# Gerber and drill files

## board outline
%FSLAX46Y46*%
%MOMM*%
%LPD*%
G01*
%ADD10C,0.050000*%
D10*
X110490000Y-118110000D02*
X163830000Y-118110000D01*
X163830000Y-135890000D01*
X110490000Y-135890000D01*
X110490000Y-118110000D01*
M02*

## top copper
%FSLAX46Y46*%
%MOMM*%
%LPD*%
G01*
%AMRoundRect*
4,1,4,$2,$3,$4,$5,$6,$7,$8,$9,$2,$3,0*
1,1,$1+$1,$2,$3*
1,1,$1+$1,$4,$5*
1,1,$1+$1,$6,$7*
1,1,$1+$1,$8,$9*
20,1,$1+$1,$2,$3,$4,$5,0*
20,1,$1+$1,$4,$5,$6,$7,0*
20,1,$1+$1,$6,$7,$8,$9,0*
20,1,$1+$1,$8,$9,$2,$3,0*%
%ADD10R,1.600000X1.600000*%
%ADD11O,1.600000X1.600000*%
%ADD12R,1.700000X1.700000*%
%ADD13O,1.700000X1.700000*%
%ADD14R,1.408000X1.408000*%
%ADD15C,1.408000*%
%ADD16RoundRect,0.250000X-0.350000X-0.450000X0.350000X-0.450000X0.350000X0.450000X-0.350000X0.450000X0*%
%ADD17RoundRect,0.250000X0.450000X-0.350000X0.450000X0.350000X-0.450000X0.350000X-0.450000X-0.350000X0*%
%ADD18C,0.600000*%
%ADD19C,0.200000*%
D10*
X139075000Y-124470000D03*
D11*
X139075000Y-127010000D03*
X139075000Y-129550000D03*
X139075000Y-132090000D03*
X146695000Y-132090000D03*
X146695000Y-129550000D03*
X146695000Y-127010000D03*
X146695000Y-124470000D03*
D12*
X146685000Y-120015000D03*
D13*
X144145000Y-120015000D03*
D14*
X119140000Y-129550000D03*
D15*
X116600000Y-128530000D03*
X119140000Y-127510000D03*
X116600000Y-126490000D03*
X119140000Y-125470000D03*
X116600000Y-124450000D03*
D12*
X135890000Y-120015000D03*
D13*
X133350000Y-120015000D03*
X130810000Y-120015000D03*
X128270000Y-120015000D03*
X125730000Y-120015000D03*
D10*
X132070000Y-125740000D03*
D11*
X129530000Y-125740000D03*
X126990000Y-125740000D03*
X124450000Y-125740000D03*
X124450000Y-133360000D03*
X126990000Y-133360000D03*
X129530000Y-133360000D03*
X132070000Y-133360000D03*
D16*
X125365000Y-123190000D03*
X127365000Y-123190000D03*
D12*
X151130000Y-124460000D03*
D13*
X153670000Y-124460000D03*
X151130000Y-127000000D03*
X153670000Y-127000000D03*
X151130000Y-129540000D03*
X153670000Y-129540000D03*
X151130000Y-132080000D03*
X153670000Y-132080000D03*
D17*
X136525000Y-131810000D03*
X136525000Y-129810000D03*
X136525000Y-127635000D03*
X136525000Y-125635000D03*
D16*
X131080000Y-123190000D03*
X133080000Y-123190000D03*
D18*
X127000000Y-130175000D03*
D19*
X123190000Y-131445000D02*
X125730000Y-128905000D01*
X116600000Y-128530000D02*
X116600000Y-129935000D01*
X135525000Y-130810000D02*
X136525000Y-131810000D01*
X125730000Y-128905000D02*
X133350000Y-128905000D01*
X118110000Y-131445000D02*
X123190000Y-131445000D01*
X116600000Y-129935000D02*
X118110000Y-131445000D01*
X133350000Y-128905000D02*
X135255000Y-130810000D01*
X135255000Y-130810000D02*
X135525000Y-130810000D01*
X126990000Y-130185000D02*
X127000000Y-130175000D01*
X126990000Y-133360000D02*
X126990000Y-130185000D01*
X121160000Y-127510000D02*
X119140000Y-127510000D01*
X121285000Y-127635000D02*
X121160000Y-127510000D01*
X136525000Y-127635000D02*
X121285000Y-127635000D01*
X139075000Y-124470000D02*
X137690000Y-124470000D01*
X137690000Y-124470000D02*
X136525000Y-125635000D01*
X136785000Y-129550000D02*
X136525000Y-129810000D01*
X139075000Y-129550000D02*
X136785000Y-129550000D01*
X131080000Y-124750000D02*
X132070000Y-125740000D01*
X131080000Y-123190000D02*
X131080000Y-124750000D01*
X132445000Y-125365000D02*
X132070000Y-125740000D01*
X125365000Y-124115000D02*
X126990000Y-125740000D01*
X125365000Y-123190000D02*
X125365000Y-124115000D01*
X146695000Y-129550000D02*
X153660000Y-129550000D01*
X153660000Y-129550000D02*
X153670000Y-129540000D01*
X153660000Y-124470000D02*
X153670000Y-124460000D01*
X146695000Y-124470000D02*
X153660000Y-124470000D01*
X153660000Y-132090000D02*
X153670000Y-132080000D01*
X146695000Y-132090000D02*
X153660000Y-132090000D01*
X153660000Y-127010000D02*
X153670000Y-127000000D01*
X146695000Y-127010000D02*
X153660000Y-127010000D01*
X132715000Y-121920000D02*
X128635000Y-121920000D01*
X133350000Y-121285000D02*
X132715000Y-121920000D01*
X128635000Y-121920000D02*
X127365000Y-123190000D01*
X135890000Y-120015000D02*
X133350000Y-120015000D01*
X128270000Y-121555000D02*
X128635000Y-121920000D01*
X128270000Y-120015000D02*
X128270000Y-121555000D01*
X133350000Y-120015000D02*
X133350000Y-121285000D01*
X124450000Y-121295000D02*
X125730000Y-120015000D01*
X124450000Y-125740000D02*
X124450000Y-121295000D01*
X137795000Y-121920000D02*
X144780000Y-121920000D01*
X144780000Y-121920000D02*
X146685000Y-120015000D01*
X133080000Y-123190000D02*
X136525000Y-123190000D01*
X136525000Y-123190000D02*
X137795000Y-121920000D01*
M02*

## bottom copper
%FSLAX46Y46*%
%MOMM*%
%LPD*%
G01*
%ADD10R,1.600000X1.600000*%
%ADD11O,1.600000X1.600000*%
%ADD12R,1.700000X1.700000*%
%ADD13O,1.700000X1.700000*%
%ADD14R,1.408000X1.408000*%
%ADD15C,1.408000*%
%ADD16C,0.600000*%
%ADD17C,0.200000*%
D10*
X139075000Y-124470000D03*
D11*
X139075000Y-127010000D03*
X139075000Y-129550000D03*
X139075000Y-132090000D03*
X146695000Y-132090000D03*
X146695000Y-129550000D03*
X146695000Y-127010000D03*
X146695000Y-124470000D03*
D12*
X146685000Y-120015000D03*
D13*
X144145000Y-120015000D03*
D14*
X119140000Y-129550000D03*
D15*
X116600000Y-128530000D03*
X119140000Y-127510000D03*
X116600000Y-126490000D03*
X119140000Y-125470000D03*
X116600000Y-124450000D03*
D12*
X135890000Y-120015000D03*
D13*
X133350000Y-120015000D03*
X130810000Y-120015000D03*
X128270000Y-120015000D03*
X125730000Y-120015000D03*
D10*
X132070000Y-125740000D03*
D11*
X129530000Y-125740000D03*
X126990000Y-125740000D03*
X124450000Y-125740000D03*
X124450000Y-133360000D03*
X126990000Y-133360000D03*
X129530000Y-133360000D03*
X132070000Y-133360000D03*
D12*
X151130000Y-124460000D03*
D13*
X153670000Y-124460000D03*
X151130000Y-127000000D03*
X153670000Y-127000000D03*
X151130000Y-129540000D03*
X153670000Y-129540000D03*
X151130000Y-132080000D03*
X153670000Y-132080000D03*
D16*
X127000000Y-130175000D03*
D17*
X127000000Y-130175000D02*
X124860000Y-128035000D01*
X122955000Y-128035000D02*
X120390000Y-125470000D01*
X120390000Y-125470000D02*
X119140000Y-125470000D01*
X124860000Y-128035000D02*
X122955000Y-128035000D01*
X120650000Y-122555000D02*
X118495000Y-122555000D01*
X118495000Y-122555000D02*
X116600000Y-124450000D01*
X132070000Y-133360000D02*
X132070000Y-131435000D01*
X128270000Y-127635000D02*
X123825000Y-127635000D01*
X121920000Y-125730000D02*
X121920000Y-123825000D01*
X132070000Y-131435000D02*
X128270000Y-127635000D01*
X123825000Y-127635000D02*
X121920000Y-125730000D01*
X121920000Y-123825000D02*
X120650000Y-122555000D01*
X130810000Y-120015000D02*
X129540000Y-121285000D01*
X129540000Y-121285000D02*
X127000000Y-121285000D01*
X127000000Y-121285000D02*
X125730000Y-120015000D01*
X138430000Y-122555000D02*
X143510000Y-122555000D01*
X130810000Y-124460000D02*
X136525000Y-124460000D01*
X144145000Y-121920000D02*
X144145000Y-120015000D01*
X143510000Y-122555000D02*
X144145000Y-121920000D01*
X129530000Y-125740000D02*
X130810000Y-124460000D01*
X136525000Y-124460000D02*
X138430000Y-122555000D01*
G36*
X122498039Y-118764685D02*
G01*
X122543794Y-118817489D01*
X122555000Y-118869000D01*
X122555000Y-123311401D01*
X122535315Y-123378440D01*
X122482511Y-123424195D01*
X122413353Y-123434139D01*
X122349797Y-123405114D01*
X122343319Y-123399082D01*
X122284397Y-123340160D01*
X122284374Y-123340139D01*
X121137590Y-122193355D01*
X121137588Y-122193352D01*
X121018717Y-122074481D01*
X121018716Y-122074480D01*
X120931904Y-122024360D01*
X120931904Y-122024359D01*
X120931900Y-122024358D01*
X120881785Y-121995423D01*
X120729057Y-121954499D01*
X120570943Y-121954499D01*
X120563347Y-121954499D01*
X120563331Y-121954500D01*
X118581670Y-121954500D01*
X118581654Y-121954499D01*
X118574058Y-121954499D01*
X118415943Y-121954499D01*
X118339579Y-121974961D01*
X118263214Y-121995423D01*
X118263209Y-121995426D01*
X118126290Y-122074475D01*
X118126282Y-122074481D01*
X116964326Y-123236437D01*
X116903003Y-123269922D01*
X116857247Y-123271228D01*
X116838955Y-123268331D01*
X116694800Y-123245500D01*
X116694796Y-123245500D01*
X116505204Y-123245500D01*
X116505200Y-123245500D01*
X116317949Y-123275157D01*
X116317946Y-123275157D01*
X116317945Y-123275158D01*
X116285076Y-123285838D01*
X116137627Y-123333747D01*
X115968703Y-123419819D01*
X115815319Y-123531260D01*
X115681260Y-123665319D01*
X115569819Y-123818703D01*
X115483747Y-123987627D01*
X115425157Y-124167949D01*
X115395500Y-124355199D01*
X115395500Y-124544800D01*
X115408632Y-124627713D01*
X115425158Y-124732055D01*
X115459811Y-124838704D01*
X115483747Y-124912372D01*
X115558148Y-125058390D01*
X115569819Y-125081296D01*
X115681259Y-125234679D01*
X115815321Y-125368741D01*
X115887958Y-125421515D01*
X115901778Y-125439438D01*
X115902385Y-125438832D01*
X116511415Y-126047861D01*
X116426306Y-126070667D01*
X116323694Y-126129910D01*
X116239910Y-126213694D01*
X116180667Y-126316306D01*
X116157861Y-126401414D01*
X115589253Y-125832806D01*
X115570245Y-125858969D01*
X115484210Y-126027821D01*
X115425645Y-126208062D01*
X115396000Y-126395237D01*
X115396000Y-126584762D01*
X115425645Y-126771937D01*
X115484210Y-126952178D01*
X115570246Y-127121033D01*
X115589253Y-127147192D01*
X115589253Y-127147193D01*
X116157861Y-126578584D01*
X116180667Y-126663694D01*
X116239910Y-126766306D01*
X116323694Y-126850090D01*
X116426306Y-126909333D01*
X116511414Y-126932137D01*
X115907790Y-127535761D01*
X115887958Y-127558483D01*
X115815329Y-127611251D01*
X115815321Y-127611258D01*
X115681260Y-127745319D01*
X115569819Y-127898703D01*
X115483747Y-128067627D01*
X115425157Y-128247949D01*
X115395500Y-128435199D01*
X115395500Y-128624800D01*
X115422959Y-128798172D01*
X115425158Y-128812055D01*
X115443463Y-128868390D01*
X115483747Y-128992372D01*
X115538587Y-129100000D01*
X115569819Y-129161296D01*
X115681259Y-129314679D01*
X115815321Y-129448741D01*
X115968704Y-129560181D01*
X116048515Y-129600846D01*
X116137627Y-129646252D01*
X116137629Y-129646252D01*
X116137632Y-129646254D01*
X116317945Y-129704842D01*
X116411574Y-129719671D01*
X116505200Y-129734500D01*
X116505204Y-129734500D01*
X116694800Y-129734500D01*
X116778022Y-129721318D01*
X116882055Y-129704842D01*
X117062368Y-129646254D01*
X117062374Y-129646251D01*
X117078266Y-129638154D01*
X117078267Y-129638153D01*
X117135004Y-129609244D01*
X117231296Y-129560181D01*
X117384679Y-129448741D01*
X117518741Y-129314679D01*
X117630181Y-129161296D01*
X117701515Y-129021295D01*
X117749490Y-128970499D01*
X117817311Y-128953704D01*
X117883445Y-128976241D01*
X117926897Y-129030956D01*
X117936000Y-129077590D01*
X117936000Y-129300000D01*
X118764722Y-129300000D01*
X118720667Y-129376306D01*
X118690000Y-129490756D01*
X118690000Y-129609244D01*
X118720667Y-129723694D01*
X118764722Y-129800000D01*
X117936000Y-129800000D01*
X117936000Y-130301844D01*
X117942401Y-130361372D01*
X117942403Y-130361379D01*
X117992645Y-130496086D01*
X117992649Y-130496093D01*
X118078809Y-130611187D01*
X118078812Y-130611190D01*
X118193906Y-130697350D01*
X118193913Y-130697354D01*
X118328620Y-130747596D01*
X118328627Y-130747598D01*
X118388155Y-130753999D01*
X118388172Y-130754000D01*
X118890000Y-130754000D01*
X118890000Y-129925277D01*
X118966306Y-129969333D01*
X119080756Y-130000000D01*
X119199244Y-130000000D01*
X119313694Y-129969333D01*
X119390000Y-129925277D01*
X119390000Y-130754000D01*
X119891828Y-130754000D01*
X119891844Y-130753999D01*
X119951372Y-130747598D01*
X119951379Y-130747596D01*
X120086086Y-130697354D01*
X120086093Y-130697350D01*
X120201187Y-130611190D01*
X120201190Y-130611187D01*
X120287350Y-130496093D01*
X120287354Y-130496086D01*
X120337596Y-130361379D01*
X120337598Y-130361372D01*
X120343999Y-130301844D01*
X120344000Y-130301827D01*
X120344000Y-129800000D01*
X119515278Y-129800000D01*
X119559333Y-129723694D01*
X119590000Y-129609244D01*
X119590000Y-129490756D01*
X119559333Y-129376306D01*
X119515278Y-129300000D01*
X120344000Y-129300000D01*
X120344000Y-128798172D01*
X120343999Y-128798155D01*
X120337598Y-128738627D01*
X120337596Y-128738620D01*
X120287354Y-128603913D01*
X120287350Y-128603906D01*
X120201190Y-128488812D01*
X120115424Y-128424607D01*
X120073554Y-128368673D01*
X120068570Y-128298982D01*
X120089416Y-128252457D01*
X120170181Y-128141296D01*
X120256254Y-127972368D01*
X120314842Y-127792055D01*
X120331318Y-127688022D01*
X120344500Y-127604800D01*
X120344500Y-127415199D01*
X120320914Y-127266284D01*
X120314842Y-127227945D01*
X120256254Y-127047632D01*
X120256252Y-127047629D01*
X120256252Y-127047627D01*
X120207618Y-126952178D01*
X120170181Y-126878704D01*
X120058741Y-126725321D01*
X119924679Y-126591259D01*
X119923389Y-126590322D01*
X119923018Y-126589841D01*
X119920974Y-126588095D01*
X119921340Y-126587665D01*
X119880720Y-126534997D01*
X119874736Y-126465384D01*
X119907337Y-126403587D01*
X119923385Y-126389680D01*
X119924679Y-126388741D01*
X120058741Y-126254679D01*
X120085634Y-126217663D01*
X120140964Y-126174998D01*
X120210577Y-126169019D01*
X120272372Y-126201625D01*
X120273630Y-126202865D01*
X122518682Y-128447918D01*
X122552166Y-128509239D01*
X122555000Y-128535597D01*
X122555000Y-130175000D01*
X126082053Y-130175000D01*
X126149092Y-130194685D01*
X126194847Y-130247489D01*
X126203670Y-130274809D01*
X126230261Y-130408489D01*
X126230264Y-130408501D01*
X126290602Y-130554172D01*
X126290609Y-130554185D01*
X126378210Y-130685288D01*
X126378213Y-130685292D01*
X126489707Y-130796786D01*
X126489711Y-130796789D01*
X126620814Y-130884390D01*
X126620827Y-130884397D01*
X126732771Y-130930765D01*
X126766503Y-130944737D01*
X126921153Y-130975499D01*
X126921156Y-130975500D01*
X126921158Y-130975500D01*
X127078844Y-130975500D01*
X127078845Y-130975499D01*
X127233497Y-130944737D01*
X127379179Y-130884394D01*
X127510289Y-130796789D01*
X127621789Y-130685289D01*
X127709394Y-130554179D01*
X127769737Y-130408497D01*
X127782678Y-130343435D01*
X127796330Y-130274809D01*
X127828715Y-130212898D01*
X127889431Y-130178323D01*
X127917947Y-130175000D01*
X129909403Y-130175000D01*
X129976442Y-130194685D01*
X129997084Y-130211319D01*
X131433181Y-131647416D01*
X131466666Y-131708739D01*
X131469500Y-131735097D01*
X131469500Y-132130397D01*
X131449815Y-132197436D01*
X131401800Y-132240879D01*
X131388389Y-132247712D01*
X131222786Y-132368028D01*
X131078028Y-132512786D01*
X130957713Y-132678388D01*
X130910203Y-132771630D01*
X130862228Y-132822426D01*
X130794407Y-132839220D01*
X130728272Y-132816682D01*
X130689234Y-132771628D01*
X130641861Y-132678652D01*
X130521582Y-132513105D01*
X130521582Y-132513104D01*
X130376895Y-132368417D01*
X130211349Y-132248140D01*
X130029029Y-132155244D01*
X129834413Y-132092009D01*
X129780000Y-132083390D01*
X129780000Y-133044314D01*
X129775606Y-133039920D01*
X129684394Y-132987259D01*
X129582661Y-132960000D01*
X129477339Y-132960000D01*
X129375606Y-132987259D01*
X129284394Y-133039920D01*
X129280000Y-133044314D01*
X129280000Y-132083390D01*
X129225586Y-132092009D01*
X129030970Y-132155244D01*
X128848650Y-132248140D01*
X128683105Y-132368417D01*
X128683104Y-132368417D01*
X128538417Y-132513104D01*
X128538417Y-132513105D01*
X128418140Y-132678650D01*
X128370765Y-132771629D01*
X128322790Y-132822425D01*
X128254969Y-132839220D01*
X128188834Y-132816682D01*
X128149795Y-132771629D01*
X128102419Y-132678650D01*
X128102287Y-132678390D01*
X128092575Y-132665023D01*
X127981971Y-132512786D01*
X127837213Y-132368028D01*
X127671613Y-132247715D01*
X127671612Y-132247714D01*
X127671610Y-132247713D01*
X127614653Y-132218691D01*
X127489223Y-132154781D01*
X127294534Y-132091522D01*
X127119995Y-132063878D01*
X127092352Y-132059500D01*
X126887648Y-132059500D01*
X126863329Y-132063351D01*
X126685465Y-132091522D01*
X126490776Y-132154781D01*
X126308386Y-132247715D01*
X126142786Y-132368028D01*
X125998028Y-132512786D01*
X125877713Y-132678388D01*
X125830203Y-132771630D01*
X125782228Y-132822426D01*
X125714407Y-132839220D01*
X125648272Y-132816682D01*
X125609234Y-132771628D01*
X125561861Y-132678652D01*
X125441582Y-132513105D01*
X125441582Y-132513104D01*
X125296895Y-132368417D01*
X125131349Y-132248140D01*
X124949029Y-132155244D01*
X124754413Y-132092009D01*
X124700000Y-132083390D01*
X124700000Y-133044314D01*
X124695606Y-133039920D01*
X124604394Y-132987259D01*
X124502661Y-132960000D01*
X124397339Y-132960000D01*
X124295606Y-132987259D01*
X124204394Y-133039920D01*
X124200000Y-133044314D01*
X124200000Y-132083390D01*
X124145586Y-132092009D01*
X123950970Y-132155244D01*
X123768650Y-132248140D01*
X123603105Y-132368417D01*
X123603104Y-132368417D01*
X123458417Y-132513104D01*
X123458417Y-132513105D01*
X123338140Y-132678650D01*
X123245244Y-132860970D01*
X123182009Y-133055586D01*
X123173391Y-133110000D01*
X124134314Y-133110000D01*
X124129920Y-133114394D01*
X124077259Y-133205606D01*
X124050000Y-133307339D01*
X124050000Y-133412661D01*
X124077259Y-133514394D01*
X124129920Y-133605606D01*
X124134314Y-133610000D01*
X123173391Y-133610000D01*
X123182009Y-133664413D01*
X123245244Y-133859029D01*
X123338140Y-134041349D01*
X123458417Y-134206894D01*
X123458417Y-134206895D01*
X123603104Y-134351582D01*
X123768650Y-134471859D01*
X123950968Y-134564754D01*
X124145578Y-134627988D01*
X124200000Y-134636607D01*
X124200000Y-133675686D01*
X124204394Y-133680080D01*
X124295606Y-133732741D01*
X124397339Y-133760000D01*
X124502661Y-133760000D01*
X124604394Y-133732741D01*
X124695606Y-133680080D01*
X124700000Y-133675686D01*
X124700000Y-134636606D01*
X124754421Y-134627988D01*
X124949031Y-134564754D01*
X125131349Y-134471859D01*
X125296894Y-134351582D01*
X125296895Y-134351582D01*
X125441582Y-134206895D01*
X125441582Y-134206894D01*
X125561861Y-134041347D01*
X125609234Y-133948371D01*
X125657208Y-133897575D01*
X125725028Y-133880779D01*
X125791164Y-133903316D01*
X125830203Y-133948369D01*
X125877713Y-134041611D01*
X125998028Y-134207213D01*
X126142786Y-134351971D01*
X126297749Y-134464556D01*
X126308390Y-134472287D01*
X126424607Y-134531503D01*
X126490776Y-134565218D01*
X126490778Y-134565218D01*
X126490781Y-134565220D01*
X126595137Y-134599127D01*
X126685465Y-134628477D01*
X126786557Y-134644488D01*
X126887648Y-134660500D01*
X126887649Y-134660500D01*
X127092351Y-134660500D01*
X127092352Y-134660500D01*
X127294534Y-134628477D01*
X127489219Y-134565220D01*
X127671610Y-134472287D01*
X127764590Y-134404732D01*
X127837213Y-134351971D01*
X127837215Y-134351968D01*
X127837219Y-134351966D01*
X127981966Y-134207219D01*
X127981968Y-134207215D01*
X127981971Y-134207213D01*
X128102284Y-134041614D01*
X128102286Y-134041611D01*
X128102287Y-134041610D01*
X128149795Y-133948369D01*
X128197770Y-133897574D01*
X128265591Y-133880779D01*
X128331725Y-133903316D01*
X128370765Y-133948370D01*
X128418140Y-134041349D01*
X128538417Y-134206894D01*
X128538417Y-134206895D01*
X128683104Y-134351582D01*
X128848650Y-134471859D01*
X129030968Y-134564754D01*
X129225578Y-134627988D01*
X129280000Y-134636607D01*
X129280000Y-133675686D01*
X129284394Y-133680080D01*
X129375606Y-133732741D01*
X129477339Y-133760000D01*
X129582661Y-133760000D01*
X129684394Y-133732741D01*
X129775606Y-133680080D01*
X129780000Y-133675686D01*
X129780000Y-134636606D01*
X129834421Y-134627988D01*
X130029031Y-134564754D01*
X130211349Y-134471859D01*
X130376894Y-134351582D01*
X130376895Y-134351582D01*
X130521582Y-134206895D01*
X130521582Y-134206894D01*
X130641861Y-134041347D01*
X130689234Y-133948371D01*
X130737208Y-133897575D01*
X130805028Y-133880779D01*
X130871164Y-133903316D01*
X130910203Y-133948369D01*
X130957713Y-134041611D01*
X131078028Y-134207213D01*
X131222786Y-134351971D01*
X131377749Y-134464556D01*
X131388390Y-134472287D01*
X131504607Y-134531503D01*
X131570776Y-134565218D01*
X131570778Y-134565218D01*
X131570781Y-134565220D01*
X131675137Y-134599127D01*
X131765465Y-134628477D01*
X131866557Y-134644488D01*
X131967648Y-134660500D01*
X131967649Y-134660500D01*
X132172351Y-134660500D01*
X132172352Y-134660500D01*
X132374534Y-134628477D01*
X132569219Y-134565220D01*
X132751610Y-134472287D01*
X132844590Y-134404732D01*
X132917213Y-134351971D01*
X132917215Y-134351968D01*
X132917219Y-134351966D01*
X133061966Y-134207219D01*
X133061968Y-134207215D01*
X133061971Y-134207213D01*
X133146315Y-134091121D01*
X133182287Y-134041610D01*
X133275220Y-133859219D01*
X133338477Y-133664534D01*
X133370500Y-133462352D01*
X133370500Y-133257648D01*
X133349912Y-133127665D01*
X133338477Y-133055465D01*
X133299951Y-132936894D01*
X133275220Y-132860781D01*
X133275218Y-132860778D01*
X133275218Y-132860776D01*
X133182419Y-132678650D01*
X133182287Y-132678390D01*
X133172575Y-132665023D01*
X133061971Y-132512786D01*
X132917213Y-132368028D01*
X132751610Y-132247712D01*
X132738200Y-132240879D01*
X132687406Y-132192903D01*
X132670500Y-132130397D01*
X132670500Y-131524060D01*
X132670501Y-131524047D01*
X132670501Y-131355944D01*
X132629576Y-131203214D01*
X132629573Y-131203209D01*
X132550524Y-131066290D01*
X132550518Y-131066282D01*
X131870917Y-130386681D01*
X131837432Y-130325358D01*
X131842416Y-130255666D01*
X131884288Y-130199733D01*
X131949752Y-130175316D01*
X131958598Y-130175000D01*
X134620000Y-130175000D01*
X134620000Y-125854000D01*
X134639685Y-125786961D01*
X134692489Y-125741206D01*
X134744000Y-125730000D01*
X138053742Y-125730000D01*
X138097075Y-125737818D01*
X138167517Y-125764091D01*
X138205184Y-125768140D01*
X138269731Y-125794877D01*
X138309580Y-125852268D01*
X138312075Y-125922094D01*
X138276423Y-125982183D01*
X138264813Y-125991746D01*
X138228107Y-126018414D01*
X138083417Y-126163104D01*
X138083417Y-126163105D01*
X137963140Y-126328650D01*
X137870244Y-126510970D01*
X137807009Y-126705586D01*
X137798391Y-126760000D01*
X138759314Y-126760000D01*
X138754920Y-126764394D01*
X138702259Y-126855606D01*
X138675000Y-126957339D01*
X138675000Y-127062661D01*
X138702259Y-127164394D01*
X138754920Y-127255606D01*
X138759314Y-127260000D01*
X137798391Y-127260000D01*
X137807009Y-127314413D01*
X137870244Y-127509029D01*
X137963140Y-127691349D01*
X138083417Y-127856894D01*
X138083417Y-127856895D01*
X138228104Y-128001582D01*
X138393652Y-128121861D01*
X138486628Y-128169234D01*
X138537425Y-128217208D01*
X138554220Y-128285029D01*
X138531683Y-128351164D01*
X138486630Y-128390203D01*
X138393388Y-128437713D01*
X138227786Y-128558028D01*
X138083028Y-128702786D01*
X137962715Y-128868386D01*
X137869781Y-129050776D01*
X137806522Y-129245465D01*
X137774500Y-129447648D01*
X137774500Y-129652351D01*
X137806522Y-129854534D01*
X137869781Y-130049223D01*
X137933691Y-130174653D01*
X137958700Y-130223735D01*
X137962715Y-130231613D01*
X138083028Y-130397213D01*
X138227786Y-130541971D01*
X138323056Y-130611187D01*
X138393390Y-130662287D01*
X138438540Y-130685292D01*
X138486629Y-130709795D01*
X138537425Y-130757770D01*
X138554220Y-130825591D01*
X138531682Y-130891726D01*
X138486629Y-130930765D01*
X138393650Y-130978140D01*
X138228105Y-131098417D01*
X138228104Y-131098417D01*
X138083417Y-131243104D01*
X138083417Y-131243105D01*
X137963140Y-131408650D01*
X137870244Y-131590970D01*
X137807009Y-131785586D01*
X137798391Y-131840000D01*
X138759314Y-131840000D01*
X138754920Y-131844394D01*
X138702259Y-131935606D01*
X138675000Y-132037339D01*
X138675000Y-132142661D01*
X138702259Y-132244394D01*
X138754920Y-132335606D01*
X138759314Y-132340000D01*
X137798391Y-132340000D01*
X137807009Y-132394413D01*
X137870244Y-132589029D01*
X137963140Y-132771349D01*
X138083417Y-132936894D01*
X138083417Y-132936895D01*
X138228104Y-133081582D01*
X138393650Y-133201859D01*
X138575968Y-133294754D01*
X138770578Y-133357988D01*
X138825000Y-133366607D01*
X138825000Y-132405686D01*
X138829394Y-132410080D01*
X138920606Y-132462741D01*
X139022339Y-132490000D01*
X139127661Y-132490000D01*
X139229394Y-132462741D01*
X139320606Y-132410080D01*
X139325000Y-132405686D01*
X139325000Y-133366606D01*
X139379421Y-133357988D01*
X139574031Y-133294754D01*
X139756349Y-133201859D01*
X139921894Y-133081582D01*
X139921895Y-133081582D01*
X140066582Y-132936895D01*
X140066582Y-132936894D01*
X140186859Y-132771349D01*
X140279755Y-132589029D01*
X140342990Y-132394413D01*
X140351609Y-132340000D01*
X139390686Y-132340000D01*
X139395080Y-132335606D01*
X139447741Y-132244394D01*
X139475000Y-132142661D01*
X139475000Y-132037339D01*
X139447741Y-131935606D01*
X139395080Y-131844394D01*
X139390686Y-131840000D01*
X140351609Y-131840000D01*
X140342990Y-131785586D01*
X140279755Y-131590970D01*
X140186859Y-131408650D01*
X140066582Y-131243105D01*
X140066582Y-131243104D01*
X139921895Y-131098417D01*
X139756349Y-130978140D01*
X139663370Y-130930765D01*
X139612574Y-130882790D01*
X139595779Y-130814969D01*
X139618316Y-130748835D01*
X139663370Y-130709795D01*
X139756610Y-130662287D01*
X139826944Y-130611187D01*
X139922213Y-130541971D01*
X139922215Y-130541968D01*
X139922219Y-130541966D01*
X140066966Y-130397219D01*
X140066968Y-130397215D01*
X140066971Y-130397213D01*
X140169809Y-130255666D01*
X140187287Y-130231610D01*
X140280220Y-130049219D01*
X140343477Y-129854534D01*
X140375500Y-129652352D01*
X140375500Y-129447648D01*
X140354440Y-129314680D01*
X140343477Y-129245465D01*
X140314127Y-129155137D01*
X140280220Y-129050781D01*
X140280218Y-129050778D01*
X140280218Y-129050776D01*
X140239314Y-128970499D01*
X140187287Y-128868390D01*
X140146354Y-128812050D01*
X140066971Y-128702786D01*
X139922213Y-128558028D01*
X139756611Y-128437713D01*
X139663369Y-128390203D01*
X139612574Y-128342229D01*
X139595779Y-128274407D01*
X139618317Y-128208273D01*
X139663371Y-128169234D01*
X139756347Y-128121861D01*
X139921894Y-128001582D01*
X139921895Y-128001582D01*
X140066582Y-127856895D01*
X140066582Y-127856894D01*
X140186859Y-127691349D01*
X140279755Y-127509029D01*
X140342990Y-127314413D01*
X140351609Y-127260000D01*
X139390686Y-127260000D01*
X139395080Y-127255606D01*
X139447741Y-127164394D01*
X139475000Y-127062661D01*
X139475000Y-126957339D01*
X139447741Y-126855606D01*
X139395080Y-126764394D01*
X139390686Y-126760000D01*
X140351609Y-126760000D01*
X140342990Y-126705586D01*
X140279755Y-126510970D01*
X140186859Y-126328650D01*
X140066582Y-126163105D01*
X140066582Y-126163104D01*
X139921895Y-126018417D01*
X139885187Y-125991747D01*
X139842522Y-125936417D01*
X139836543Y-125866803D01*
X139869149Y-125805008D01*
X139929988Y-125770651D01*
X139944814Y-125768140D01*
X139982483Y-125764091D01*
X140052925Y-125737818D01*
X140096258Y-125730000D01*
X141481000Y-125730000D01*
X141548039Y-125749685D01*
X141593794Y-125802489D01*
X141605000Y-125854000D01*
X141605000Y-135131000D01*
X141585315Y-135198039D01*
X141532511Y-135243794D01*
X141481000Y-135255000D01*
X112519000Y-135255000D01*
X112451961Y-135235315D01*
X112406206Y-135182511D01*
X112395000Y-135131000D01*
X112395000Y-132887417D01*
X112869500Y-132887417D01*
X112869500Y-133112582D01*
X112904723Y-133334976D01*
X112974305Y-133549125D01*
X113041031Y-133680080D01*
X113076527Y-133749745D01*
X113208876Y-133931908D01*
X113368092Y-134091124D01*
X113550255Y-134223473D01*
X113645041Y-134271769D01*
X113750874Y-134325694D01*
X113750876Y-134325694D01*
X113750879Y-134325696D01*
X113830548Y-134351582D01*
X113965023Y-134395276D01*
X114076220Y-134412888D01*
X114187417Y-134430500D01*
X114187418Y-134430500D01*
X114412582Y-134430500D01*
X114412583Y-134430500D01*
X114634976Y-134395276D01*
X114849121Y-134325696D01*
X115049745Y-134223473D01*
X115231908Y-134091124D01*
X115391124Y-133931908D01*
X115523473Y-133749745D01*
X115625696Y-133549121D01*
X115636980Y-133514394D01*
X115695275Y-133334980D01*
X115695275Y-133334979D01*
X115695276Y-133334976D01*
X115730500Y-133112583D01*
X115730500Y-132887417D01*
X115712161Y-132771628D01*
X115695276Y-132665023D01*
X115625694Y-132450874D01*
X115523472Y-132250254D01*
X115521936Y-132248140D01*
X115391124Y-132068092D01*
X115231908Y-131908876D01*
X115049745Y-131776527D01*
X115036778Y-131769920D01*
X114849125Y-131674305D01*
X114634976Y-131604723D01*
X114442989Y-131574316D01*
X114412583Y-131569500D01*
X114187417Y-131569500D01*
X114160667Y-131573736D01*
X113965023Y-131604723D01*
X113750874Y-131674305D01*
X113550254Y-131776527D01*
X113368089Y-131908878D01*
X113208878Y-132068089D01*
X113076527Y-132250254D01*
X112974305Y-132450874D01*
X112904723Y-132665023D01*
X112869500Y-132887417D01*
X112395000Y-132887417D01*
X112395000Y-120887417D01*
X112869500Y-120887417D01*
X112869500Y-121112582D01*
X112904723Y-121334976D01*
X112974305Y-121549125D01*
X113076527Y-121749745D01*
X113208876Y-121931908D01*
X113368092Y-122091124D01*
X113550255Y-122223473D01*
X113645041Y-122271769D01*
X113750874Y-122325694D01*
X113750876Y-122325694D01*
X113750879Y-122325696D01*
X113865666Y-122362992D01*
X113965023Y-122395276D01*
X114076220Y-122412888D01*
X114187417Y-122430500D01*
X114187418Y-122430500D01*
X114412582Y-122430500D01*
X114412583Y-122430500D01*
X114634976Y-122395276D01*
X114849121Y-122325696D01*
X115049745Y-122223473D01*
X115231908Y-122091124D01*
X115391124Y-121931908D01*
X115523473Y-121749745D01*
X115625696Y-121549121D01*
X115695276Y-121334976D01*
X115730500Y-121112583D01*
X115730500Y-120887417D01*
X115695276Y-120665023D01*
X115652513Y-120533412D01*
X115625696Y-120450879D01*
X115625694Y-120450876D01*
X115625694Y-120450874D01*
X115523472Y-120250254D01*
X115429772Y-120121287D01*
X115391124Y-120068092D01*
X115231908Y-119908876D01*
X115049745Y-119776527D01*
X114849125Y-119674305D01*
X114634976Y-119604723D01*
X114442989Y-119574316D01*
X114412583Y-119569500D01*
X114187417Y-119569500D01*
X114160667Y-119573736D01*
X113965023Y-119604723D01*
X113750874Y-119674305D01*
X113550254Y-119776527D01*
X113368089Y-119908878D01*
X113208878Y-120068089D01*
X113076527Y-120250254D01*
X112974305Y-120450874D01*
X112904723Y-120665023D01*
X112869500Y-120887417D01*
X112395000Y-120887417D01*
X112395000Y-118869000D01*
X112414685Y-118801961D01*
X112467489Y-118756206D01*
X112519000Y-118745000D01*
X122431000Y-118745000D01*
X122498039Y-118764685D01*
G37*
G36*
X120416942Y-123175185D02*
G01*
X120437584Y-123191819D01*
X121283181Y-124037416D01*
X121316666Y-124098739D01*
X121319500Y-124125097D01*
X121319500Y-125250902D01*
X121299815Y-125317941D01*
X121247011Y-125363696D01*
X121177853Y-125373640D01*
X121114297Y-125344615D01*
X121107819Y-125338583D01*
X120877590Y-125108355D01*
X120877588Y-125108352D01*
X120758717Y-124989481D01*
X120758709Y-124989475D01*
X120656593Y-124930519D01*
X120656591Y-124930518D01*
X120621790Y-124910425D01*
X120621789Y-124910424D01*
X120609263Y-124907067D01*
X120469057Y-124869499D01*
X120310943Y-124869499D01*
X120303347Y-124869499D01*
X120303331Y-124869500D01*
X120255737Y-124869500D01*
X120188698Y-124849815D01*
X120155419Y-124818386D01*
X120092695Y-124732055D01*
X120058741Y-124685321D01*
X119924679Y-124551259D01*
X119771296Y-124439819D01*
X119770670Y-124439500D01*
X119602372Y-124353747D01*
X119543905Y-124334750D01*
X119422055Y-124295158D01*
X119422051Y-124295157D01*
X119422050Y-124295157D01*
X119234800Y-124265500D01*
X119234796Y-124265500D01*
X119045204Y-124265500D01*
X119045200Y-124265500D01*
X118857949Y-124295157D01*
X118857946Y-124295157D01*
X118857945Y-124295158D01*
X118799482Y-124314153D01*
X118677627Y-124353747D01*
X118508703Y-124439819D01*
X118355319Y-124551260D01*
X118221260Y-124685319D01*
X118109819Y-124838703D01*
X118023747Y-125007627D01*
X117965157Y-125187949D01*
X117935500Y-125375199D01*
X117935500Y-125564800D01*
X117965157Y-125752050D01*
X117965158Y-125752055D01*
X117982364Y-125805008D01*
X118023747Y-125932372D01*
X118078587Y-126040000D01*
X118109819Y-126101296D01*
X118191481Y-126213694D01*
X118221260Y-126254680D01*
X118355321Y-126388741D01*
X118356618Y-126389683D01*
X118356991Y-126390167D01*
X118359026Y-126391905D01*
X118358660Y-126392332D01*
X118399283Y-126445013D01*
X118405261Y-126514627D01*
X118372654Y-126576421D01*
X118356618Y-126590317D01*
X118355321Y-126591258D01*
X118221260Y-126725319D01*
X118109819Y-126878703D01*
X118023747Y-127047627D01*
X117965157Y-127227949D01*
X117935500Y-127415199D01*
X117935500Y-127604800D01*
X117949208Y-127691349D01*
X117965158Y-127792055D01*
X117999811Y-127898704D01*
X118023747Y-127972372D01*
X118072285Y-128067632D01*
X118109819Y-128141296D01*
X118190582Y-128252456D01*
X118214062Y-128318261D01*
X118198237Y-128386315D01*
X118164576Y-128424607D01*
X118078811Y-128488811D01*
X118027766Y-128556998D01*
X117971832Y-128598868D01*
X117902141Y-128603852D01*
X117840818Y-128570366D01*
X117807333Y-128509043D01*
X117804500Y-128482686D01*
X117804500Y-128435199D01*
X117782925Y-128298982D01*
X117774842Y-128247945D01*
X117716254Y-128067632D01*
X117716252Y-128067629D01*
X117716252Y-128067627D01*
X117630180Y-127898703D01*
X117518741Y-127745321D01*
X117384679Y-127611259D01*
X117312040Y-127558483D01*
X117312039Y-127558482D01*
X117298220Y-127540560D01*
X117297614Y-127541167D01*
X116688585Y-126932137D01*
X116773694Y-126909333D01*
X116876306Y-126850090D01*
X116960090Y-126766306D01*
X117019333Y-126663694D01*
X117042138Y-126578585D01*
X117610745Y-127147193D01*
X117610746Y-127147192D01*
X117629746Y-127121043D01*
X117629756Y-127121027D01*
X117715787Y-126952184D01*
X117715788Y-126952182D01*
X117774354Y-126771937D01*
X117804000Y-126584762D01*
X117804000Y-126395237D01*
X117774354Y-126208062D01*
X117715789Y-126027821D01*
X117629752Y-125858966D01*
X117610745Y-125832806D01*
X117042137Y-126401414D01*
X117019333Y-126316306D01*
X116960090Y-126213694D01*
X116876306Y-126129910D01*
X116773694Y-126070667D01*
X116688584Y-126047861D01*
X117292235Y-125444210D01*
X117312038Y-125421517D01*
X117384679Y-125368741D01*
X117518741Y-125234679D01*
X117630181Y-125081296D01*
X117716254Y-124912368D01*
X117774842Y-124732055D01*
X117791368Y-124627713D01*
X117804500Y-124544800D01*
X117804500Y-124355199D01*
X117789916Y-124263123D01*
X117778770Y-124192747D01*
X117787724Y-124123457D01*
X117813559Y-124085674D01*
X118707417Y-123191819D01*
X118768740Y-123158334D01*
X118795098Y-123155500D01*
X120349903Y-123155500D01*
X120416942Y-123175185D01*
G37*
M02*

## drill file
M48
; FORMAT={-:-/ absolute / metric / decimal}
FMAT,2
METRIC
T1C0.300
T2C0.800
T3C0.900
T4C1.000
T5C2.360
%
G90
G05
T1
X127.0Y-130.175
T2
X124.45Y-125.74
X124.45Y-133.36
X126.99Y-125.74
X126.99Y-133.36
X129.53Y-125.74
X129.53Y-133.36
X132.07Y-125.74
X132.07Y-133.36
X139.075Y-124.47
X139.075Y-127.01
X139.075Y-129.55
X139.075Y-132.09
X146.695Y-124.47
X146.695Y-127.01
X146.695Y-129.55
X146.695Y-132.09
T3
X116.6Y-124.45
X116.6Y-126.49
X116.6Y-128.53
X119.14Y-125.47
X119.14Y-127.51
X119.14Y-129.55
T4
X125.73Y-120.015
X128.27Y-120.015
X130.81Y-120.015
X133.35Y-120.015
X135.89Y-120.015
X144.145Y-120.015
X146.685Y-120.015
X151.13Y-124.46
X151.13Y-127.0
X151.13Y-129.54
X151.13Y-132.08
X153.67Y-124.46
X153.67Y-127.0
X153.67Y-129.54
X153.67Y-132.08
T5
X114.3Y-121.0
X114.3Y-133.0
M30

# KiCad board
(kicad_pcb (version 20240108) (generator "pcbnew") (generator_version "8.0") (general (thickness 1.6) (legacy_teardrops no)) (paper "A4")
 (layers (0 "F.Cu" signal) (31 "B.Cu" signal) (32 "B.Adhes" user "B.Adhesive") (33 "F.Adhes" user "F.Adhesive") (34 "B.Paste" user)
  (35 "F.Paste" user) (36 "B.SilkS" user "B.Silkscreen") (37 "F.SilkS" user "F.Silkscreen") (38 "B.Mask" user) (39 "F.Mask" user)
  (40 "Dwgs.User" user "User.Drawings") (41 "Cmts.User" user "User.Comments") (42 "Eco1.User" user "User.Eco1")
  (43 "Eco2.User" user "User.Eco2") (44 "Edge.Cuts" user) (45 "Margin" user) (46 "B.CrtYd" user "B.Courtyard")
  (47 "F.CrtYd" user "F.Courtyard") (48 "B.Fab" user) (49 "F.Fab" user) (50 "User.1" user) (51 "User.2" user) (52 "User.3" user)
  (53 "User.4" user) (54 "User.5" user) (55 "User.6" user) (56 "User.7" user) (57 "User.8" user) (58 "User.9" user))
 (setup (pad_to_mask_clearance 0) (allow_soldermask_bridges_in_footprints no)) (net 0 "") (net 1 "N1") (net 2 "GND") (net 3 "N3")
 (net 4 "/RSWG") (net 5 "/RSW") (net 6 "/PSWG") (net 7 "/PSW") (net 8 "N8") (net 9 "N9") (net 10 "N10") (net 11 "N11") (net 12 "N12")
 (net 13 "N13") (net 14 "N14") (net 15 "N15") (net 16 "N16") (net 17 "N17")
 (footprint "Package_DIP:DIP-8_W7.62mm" (layer "F.Cu") (at 139.075 124.47)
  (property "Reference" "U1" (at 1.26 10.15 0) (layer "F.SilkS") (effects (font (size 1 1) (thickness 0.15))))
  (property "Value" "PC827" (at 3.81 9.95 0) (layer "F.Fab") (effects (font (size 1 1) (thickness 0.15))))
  (pad "1" thru_hole rect (at 0 0) (size 1.6 1.6) (drill 0.8) (layers "*.Cu" "*.Mask") (remove_unused_layers no) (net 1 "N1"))
  (pad "2" thru_hole oval (at 0 2.54) (size 1.6 1.6) (drill 0.8) (layers "*.Cu" "*.Mask") (remove_unused_layers no) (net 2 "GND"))
  (pad "3" thru_hole oval (at 0 5.08) (size 1.6 1.6) (drill 0.8) (layers "*.Cu" "*.Mask") (remove_unused_layers no) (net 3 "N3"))
  (pad "4" thru_hole oval (at 0 7.62) (size 1.6 1.6) (drill 0.8) (layers "*.Cu" "*.Mask") (remove_unused_layers no) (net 2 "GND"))
  (pad "5" thru_hole oval (at 7.62 7.62) (size 1.6 1.6) (drill 0.8) (layers "*.Cu" "*.Mask") (remove_unused_layers no) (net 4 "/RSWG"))
  (pad "6" thru_hole oval (at 7.62 5.08) (size 1.6 1.6) (drill 0.8) (layers "*.Cu" "*.Mask") (remove_unused_layers no) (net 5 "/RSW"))
  (pad "7" thru_hole oval (at 7.62 2.54) (size 1.6 1.6) (drill 0.8) (layers "*.Cu" "*.Mask") (remove_unused_layers no) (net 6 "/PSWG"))
  (pad "8" thru_hole oval (at 7.62 0) (size 1.6 1.6) (drill 0.8) (layers "*.Cu" "*.Mask") (remove_unused_layers no) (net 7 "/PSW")))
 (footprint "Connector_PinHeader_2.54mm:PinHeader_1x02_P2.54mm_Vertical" (layer "F.Cu") (at 146.685 120.015 -90)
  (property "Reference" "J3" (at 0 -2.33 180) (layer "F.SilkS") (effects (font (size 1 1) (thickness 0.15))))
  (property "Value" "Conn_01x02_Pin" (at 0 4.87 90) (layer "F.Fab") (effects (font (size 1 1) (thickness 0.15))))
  (pad "1" thru_hole rect (at 0 0 270) (size 1.7 1.7) (drill 1) (layers "*.Cu" "*.Mask") (remove_unused_layers no) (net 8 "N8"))
  (pad "2" thru_hole oval (at 0 2.54 270) (size 1.7 1.7) (drill 1) (layers "*.Cu" "*.Mask") (remove_unused_layers no) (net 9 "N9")))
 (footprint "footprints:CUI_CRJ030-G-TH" (layer "F.Cu") (at 114.3 127 -90)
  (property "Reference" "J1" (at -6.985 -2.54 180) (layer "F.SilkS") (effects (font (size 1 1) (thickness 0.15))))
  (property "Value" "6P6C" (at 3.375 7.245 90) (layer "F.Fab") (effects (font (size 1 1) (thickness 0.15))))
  (pad "" np_thru_hole circle (at -6 0 270) (size 2.36 2.36) (drill 2.36) (layers "*.Cu" "*.Mask"))
  (pad "" np_thru_hole circle (at 6 0 270) (size 2.36 2.36) (drill 2.36) (layers "*.Cu" "*.Mask"))
  (pad "1" thru_hole rect (at 2.55 -4.84 270) (size 1.408 1.408) (drill 0.9) (layers "*.Cu" "*.Mask") (remove_unused_layers no)
   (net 2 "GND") (solder_mask_margin 0.102))
  (pad "2" thru_hole circle (at 1.53 -2.3 270) (size 1.408 1.408) (drill 0.9) (layers "*.Cu" "*.Mask") (remove_unused_layers no)
   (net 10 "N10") (solder_mask_margin 0.102))
  (pad "3" thru_hole circle (at 0.51 -4.84 270) (size 1.408 1.408) (drill 0.9) (layers "*.Cu" "*.Mask") (remove_unused_layers no)
   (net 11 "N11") (solder_mask_margin 0.102))
  (pad "4" thru_hole circle (at -0.51 -2.3 270) (size 1.408 1.408) (drill 0.9) (layers "*.Cu" "*.Mask") (remove_unused_layers no)
   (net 2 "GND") (solder_mask_margin 0.102))
  (pad "5" thru_hole circle (at -1.53 -4.84 270) (size 1.408 1.408) (drill 0.9) (layers "*.Cu" "*.Mask") (remove_unused_layers no)
   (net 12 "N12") (solder_mask_margin 0.102))
  (pad "6" thru_hole circle (at -2.55 -2.3 270) (size 1.408 1.408) (drill 0.9) (layers "*.Cu" "*.Mask") (remove_unused_layers no)
   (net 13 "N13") (solder_mask_margin 0.102)))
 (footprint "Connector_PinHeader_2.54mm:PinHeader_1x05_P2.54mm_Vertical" (layer "F.Cu") (at 135.89 120.015 -90)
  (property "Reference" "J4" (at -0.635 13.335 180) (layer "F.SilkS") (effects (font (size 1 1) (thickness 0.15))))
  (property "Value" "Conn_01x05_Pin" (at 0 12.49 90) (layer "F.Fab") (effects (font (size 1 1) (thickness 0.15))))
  (pad "1" thru_hole rect (at 0 0 270) (size 1.7 1.7) (drill 1) (layers "*.Cu" "*.Mask") (remove_unused_layers no) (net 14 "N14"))
  (pad "2" thru_hole oval (at 0 2.54 270) (size 1.7 1.7) (drill 1) (layers "*.Cu" "*.Mask") (remove_unused_layers no) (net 14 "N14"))
  (pad "3" thru_hole oval (at 0 5.08 270) (size 1.7 1.7) (drill 1) (layers "*.Cu" "*.Mask") (remove_unused_layers no) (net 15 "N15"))
  (pad "4" thru_hole oval (at 0 7.62 270) (size 1.7 1.7) (drill 1) (layers "*.Cu" "*.Mask") (remove_unused_layers no) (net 14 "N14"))
  (pad "5" thru_hole oval (at 0 10.16 270) (size 1.7 1.7) (drill 1) (layers "*.Cu" "*.Mask") (remove_unused_layers no) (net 15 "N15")))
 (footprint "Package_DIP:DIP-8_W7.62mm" (layer "F.Cu") (at 132.07 125.74 -90)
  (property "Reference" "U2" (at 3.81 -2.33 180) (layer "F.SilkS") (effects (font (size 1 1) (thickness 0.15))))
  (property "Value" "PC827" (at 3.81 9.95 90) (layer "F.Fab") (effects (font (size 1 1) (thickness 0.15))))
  (pad "1" thru_hole rect (at 0 0 270) (size 1.6 1.6) (drill 0.8) (layers "*.Cu" "*.Mask") (remove_unused_layers no) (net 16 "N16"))
  (pad "2" thru_hole oval (at 0 2.54 270) (size 1.6 1.6) (drill 0.8) (layers "*.Cu" "*.Mask") (remove_unused_layers no) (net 9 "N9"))
  (pad "3" thru_hole oval (at 0 5.08 270) (size 1.6 1.6) (drill 0.8) (layers "*.Cu" "*.Mask") (remove_unused_layers no) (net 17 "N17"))
  (pad "4" thru_hole oval (at 0 7.62 270) (size 1.6 1.6) (drill 0.8) (layers "*.Cu" "*.Mask") (remove_unused_layers no) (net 15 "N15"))
  (pad "5" thru_hole oval (at 7.62 7.62 270) (size 1.6 1.6) (drill 0.8) (layers "*.Cu" "*.Mask") (remove_unused_layers no) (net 2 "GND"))
  (pad "6" thru_hole oval (at 7.62 5.08 270) (size 1.6 1.6) (drill 0.8) (layers "*.Cu" "*.Mask") (remove_unused_layers no) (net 12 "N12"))
  (pad "7" thru_hole oval (at 7.62 2.54 270) (size 1.6 1.6) (drill 0.8) (layers "*.Cu" "*.Mask") (remove_unused_layers no) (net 2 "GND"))
  (pad "8" thru_hole oval (at 7.62 0 270) (size 1.6 1.6) (drill 0.8) (layers "*.Cu" "*.Mask") (remove_unused_layers no) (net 13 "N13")))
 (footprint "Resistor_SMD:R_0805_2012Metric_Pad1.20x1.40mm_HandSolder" (layer "F.Cu") (at 126.365 123.19)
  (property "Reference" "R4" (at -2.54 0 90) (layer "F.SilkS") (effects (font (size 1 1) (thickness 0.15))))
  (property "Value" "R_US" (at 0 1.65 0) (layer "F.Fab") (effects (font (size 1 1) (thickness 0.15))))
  (pad "1" smd roundrect (at -1 0) (size 1.2 1.4) (layers "F.Cu" "F.Paste" "F.Mask") (roundrect_rratio 0.208333) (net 17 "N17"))
  (pad "2" smd roundrect (at 1 0) (size 1.2 1.4) (layers "F.Cu" "F.Paste" "F.Mask") (roundrect_rratio 0.208333) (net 14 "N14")))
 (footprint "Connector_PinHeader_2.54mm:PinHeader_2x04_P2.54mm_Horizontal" (layer "F.Cu") (at 151.13 124.46)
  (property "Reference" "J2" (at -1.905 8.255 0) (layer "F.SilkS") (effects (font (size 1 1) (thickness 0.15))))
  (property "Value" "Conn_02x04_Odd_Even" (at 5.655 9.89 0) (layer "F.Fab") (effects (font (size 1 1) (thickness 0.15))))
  (pad "1" thru_hole rect (at 0 0) (size 1.7 1.7) (drill 1) (layers "*.Cu" "*.Mask") (remove_unused_layers no) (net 7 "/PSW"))
  (pad "2" thru_hole oval (at 2.54 0) (size 1.7 1.7) (drill 1) (layers "*.Cu" "*.Mask") (remove_unused_layers no) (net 7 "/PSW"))
  (pad "3" thru_hole oval (at 0 2.54) (size 1.7 1.7) (drill 1) (layers "*.Cu" "*.Mask") (remove_unused_layers no) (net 6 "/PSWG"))
  (pad "4" thru_hole oval (at 2.54 2.54) (size 1.7 1.7) (drill 1) (layers "*.Cu" "*.Mask") (remove_unused_layers no) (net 6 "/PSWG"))
  (pad "5" thru_hole oval (at 0 5.08) (size 1.7 1.7) (drill 1) (layers "*.Cu" "*.Mask") (remove_unused_layers no) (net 5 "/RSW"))
  (pad "6" thru_hole oval (at 2.54 5.08) (size 1.7 1.7) (drill 1) (layers "*.Cu" "*.Mask") (remove_unused_layers no) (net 5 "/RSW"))
  (pad "7" thru_hole oval (at 0 7.62) (size 1.7 1.7) (drill 1) (layers "*.Cu" "*.Mask") (remove_unused_layers no) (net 4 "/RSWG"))
  (pad "8" thru_hole oval (at 2.54 7.62) (size 1.7 1.7) (drill 1) (layers "*.Cu" "*.Mask") (remove_unused_layers no) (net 4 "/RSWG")))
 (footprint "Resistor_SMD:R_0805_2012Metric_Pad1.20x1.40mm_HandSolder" (layer "F.Cu") (at 136.525 130.81 90)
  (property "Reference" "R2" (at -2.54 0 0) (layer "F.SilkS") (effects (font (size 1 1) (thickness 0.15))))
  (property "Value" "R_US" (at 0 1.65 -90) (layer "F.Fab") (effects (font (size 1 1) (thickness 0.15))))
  (pad "1" smd roundrect (at -1 0 90) (size 1.2 1.4) (layers "F.Cu" "F.Paste" "F.Mask") (roundrect_rratio 0.208333) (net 10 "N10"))
  (pad "2" smd roundrect (at 1 0 90) (size 1.2 1.4) (layers "F.Cu" "F.Paste" "F.Mask") (roundrect_rratio 0.208333) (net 3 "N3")))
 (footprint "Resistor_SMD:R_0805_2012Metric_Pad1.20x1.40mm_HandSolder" (layer "F.Cu") (at 136.525 126.635 90)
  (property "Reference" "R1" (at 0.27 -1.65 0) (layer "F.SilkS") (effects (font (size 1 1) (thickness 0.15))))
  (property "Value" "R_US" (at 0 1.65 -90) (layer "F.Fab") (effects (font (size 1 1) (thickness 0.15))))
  (pad "1" smd roundrect (at -1 0 90) (size 1.2 1.4) (layers "F.Cu" "F.Paste" "F.Mask") (roundrect_rratio 0.208333) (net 11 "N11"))
  (pad "2" smd roundrect (at 1 0 90) (size 1.2 1.4) (layers "F.Cu" "F.Paste" "F.Mask") (roundrect_rratio 0.208333) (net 1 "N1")))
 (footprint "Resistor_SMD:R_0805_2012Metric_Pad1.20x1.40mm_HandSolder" (layer "F.Cu") (at 132.08 123.19)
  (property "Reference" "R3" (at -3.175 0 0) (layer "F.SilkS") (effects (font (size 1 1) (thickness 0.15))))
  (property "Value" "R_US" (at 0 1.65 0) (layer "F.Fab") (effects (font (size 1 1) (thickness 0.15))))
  (pad "1" smd roundrect (at -1 0) (size 1.2 1.4) (layers "F.Cu" "F.Paste" "F.Mask") (roundrect_rratio 0.208333) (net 16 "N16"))
  (pad "2" smd roundrect (at 1 0) (size 1.2 1.4) (layers "F.Cu" "F.Paste" "F.Mask") (roundrect_rratio 0.208333) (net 8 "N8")))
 (gr_rect (start 110.49 118.11) (end 163.83 135.89) (stroke (width 0.05) (type default)) (fill none) (layer "Edge.Cuts"))
 (segment (start 123.19 131.445) (end 125.73 128.905) (width 0.2) (layer "F.Cu") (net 10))
 (segment (start 116.6 128.53) (end 116.6 129.935) (width 0.2) (layer "F.Cu") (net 10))
 (segment (start 135.525 130.81) (end 136.525 131.81) (width 0.2) (layer "F.Cu") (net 10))
 (segment (start 125.73 128.905) (end 133.35 128.905) (width 0.2) (layer "F.Cu") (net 10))
 (segment (start 118.11 131.445) (end 123.19 131.445) (width 0.2) (layer "F.Cu") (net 10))
 (segment (start 116.6 129.935) (end 118.11 131.445) (width 0.2) (layer "F.Cu") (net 10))
 (segment (start 133.35 128.905) (end 135.255 130.81) (width 0.2) (layer "F.Cu") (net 10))
 (segment (start 135.255 130.81) (end 135.525 130.81) (width 0.2) (layer "F.Cu") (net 10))
 (segment (start 126.99 130.185) (end 127 130.175) (width 0.2) (layer "F.Cu") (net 12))
 (segment (start 126.99 133.36) (end 126.99 130.185) (width 0.2) (layer "F.Cu") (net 12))
 (via (at 127 130.175) (size 0.6) (drill 0.3) (layers "F.Cu" "B.Cu") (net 12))
 (segment (start 127 130.175) (end 124.86 128.035) (width 0.2) (layer "B.Cu") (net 12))
 (segment (start 122.955 128.035) (end 120.39 125.47) (width 0.2) (layer "B.Cu") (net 12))
 (segment (start 120.39 125.47) (end 119.14 125.47) (width 0.2) (layer "B.Cu") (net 12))
 (segment (start 124.86 128.035) (end 122.955 128.035) (width 0.2) (layer "B.Cu") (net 12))
 (segment (start 120.65 122.555) (end 118.495 122.555) (width 0.2) (layer "B.Cu") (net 13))
 (segment (start 118.495 122.555) (end 116.6 124.45) (width 0.2) (layer "B.Cu") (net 13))
 (segment (start 132.07 133.36) (end 132.07 131.435) (width 0.2) (layer "B.Cu") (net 13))
 (segment (start 128.27 127.635) (end 123.825 127.635) (width 0.2) (layer "B.Cu") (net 13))
 (segment (start 121.92 125.73) (end 121.92 123.825) (width 0.2) (layer "B.Cu") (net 13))
 (segment (start 132.07 131.435) (end 128.27 127.635) (width 0.2) (layer "B.Cu") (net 13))
 (segment (start 123.825 127.635) (end 121.92 125.73) (width 0.2) (layer "B.Cu") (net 13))
 (segment (start 121.92 123.825) (end 120.65 122.555) (width 0.2) (layer "B.Cu") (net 13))
 (segment (start 121.16 127.51) (end 119.14 127.51) (width 0.2) (layer "F.Cu") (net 11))
 (segment (start 121.285 127.635) (end 121.16 127.51) (width 0.2) (layer "F.Cu") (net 11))
 (segment (start 136.525 127.635) (end 121.285 127.635) (width 0.2) (layer "F.Cu") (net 11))
 (segment (start 139.075 124.47) (end 137.69 124.47) (width 0.2) (layer "F.Cu") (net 1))
 (segment (start 137.69 124.47) (end 136.525 125.635) (width 0.2) (layer "F.Cu") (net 1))
 (segment (start 136.785 129.55) (end 136.525 129.81) (width 0.2) (layer "F.Cu") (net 3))
 (segment (start 139.075 129.55) (end 136.785 129.55) (width 0.2) (layer "F.Cu") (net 3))
 (segment (start 131.08 124.75) (end 132.07 125.74) (width 0.2) (layer "F.Cu") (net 16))
 (segment (start 131.08 123.19) (end 131.08 124.75) (width 0.2) (layer "F.Cu") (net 16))
 (segment (start 132.445 125.365) (end 132.07 125.74) (width 0.2) (layer "F.Cu") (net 16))
 (segment (start 125.365 124.115) (end 126.99 125.74) (width 0.2) (layer "F.Cu") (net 17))
 (segment (start 125.365 123.19) (end 125.365 124.115) (width 0.2) (layer "F.Cu") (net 17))
 (segment (start 146.695 129.55) (end 153.66 129.55) (width 0.2) (layer "F.Cu") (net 5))
 (segment (start 153.66 129.55) (end 153.67 129.54) (width 0.2) (layer "F.Cu") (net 5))
 (segment (start 153.66 124.47) (end 153.67 124.46) (width 0.2) (layer "F.Cu") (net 7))
 (segment (start 146.695 124.47) (end 153.66 124.47) (width 0.2) (layer "F.Cu") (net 7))
 (segment (start 153.66 132.09) (end 153.67 132.08) (width 0.2) (layer "F.Cu") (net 4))
 (segment (start 146.695 132.09) (end 153.66 132.09) (width 0.2) (layer "F.Cu") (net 4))
 (segment (start 153.66 127.01) (end 153.67 127) (width 0.2) (layer "F.Cu") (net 6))
 (segment (start 146.695 127.01) (end 153.66 127.01) (width 0.2) (layer "F.Cu") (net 6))
 (segment (start 132.715 121.92) (end 128.635 121.92) (width 0.2) (layer "F.Cu") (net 14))
 (segment (start 133.35 121.285) (end 132.715 121.92) (width 0.2) (layer "F.Cu") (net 14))
 (segment (start 128.635 121.92) (end 127.365 123.19) (width 0.2) (layer "F.Cu") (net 14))
 (segment (start 135.89 120.015) (end 133.35 120.015) (width 0.2) (layer "F.Cu") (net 14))
 (segment (start 128.27 121.555) (end 128.635 121.92) (width 0.2) (layer "F.Cu") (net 14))
 (segment (start 128.27 120.015) (end 128.27 121.555) (width 0.2) (layer "F.Cu") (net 14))
 (segment (start 133.35 120.015) (end 133.35 121.285) (width 0.2) (layer "F.Cu") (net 14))
 (segment (start 124.45 121.295) (end 125.73 120.015) (width 0.2) (layer "F.Cu") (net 15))
 (segment (start 124.45 125.74) (end 124.45 121.295) (width 0.2) (layer "F.Cu") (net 15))
 (segment (start 130.81 120.015) (end 129.54 121.285) (width 0.2) (layer "B.Cu") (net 15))
 (segment (start 129.54 121.285) (end 127 121.285) (width 0.2) (layer "B.Cu") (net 15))
 (segment (start 127 121.285) (end 125.73 120.015) (width 0.2) (layer "B.Cu") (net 15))
 (segment (start 138.43 122.555) (end 143.51 122.555) (width 0.2) (layer "B.Cu") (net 9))
 (segment (start 130.81 124.46) (end 136.525 124.46) (width 0.2) (layer "B.Cu") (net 9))
 (segment (start 144.145 121.92) (end 144.145 120.015) (width 0.2) (layer "B.Cu") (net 9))
 (segment (start 143.51 122.555) (end 144.145 121.92) (width 0.2) (layer "B.Cu") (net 9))
 (segment (start 129.53 125.74) (end 130.81 124.46) (width 0.2) (layer "B.Cu") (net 9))
 (segment (start 136.525 124.46) (end 138.43 122.555) (width 0.2) (layer "B.Cu") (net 9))
 (segment (start 137.795 121.92) (end 144.78 121.92) (width 0.2) (layer "F.Cu") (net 8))
 (segment (start 144.78 121.92) (end 146.685 120.015) (width 0.2) (layer "F.Cu") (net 8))
 (segment (start 133.08 123.19) (end 136.525 123.19) (width 0.2) (layer "F.Cu") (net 8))
 (segment (start 136.525 123.19) (end 137.795 121.92) (width 0.2) (layer "F.Cu") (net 8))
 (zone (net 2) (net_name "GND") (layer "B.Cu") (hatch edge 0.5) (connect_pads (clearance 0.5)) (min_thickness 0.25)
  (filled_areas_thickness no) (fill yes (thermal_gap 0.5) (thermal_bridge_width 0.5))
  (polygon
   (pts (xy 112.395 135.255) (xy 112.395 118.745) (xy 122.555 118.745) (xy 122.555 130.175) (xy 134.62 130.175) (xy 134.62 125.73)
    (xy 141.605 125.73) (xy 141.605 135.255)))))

